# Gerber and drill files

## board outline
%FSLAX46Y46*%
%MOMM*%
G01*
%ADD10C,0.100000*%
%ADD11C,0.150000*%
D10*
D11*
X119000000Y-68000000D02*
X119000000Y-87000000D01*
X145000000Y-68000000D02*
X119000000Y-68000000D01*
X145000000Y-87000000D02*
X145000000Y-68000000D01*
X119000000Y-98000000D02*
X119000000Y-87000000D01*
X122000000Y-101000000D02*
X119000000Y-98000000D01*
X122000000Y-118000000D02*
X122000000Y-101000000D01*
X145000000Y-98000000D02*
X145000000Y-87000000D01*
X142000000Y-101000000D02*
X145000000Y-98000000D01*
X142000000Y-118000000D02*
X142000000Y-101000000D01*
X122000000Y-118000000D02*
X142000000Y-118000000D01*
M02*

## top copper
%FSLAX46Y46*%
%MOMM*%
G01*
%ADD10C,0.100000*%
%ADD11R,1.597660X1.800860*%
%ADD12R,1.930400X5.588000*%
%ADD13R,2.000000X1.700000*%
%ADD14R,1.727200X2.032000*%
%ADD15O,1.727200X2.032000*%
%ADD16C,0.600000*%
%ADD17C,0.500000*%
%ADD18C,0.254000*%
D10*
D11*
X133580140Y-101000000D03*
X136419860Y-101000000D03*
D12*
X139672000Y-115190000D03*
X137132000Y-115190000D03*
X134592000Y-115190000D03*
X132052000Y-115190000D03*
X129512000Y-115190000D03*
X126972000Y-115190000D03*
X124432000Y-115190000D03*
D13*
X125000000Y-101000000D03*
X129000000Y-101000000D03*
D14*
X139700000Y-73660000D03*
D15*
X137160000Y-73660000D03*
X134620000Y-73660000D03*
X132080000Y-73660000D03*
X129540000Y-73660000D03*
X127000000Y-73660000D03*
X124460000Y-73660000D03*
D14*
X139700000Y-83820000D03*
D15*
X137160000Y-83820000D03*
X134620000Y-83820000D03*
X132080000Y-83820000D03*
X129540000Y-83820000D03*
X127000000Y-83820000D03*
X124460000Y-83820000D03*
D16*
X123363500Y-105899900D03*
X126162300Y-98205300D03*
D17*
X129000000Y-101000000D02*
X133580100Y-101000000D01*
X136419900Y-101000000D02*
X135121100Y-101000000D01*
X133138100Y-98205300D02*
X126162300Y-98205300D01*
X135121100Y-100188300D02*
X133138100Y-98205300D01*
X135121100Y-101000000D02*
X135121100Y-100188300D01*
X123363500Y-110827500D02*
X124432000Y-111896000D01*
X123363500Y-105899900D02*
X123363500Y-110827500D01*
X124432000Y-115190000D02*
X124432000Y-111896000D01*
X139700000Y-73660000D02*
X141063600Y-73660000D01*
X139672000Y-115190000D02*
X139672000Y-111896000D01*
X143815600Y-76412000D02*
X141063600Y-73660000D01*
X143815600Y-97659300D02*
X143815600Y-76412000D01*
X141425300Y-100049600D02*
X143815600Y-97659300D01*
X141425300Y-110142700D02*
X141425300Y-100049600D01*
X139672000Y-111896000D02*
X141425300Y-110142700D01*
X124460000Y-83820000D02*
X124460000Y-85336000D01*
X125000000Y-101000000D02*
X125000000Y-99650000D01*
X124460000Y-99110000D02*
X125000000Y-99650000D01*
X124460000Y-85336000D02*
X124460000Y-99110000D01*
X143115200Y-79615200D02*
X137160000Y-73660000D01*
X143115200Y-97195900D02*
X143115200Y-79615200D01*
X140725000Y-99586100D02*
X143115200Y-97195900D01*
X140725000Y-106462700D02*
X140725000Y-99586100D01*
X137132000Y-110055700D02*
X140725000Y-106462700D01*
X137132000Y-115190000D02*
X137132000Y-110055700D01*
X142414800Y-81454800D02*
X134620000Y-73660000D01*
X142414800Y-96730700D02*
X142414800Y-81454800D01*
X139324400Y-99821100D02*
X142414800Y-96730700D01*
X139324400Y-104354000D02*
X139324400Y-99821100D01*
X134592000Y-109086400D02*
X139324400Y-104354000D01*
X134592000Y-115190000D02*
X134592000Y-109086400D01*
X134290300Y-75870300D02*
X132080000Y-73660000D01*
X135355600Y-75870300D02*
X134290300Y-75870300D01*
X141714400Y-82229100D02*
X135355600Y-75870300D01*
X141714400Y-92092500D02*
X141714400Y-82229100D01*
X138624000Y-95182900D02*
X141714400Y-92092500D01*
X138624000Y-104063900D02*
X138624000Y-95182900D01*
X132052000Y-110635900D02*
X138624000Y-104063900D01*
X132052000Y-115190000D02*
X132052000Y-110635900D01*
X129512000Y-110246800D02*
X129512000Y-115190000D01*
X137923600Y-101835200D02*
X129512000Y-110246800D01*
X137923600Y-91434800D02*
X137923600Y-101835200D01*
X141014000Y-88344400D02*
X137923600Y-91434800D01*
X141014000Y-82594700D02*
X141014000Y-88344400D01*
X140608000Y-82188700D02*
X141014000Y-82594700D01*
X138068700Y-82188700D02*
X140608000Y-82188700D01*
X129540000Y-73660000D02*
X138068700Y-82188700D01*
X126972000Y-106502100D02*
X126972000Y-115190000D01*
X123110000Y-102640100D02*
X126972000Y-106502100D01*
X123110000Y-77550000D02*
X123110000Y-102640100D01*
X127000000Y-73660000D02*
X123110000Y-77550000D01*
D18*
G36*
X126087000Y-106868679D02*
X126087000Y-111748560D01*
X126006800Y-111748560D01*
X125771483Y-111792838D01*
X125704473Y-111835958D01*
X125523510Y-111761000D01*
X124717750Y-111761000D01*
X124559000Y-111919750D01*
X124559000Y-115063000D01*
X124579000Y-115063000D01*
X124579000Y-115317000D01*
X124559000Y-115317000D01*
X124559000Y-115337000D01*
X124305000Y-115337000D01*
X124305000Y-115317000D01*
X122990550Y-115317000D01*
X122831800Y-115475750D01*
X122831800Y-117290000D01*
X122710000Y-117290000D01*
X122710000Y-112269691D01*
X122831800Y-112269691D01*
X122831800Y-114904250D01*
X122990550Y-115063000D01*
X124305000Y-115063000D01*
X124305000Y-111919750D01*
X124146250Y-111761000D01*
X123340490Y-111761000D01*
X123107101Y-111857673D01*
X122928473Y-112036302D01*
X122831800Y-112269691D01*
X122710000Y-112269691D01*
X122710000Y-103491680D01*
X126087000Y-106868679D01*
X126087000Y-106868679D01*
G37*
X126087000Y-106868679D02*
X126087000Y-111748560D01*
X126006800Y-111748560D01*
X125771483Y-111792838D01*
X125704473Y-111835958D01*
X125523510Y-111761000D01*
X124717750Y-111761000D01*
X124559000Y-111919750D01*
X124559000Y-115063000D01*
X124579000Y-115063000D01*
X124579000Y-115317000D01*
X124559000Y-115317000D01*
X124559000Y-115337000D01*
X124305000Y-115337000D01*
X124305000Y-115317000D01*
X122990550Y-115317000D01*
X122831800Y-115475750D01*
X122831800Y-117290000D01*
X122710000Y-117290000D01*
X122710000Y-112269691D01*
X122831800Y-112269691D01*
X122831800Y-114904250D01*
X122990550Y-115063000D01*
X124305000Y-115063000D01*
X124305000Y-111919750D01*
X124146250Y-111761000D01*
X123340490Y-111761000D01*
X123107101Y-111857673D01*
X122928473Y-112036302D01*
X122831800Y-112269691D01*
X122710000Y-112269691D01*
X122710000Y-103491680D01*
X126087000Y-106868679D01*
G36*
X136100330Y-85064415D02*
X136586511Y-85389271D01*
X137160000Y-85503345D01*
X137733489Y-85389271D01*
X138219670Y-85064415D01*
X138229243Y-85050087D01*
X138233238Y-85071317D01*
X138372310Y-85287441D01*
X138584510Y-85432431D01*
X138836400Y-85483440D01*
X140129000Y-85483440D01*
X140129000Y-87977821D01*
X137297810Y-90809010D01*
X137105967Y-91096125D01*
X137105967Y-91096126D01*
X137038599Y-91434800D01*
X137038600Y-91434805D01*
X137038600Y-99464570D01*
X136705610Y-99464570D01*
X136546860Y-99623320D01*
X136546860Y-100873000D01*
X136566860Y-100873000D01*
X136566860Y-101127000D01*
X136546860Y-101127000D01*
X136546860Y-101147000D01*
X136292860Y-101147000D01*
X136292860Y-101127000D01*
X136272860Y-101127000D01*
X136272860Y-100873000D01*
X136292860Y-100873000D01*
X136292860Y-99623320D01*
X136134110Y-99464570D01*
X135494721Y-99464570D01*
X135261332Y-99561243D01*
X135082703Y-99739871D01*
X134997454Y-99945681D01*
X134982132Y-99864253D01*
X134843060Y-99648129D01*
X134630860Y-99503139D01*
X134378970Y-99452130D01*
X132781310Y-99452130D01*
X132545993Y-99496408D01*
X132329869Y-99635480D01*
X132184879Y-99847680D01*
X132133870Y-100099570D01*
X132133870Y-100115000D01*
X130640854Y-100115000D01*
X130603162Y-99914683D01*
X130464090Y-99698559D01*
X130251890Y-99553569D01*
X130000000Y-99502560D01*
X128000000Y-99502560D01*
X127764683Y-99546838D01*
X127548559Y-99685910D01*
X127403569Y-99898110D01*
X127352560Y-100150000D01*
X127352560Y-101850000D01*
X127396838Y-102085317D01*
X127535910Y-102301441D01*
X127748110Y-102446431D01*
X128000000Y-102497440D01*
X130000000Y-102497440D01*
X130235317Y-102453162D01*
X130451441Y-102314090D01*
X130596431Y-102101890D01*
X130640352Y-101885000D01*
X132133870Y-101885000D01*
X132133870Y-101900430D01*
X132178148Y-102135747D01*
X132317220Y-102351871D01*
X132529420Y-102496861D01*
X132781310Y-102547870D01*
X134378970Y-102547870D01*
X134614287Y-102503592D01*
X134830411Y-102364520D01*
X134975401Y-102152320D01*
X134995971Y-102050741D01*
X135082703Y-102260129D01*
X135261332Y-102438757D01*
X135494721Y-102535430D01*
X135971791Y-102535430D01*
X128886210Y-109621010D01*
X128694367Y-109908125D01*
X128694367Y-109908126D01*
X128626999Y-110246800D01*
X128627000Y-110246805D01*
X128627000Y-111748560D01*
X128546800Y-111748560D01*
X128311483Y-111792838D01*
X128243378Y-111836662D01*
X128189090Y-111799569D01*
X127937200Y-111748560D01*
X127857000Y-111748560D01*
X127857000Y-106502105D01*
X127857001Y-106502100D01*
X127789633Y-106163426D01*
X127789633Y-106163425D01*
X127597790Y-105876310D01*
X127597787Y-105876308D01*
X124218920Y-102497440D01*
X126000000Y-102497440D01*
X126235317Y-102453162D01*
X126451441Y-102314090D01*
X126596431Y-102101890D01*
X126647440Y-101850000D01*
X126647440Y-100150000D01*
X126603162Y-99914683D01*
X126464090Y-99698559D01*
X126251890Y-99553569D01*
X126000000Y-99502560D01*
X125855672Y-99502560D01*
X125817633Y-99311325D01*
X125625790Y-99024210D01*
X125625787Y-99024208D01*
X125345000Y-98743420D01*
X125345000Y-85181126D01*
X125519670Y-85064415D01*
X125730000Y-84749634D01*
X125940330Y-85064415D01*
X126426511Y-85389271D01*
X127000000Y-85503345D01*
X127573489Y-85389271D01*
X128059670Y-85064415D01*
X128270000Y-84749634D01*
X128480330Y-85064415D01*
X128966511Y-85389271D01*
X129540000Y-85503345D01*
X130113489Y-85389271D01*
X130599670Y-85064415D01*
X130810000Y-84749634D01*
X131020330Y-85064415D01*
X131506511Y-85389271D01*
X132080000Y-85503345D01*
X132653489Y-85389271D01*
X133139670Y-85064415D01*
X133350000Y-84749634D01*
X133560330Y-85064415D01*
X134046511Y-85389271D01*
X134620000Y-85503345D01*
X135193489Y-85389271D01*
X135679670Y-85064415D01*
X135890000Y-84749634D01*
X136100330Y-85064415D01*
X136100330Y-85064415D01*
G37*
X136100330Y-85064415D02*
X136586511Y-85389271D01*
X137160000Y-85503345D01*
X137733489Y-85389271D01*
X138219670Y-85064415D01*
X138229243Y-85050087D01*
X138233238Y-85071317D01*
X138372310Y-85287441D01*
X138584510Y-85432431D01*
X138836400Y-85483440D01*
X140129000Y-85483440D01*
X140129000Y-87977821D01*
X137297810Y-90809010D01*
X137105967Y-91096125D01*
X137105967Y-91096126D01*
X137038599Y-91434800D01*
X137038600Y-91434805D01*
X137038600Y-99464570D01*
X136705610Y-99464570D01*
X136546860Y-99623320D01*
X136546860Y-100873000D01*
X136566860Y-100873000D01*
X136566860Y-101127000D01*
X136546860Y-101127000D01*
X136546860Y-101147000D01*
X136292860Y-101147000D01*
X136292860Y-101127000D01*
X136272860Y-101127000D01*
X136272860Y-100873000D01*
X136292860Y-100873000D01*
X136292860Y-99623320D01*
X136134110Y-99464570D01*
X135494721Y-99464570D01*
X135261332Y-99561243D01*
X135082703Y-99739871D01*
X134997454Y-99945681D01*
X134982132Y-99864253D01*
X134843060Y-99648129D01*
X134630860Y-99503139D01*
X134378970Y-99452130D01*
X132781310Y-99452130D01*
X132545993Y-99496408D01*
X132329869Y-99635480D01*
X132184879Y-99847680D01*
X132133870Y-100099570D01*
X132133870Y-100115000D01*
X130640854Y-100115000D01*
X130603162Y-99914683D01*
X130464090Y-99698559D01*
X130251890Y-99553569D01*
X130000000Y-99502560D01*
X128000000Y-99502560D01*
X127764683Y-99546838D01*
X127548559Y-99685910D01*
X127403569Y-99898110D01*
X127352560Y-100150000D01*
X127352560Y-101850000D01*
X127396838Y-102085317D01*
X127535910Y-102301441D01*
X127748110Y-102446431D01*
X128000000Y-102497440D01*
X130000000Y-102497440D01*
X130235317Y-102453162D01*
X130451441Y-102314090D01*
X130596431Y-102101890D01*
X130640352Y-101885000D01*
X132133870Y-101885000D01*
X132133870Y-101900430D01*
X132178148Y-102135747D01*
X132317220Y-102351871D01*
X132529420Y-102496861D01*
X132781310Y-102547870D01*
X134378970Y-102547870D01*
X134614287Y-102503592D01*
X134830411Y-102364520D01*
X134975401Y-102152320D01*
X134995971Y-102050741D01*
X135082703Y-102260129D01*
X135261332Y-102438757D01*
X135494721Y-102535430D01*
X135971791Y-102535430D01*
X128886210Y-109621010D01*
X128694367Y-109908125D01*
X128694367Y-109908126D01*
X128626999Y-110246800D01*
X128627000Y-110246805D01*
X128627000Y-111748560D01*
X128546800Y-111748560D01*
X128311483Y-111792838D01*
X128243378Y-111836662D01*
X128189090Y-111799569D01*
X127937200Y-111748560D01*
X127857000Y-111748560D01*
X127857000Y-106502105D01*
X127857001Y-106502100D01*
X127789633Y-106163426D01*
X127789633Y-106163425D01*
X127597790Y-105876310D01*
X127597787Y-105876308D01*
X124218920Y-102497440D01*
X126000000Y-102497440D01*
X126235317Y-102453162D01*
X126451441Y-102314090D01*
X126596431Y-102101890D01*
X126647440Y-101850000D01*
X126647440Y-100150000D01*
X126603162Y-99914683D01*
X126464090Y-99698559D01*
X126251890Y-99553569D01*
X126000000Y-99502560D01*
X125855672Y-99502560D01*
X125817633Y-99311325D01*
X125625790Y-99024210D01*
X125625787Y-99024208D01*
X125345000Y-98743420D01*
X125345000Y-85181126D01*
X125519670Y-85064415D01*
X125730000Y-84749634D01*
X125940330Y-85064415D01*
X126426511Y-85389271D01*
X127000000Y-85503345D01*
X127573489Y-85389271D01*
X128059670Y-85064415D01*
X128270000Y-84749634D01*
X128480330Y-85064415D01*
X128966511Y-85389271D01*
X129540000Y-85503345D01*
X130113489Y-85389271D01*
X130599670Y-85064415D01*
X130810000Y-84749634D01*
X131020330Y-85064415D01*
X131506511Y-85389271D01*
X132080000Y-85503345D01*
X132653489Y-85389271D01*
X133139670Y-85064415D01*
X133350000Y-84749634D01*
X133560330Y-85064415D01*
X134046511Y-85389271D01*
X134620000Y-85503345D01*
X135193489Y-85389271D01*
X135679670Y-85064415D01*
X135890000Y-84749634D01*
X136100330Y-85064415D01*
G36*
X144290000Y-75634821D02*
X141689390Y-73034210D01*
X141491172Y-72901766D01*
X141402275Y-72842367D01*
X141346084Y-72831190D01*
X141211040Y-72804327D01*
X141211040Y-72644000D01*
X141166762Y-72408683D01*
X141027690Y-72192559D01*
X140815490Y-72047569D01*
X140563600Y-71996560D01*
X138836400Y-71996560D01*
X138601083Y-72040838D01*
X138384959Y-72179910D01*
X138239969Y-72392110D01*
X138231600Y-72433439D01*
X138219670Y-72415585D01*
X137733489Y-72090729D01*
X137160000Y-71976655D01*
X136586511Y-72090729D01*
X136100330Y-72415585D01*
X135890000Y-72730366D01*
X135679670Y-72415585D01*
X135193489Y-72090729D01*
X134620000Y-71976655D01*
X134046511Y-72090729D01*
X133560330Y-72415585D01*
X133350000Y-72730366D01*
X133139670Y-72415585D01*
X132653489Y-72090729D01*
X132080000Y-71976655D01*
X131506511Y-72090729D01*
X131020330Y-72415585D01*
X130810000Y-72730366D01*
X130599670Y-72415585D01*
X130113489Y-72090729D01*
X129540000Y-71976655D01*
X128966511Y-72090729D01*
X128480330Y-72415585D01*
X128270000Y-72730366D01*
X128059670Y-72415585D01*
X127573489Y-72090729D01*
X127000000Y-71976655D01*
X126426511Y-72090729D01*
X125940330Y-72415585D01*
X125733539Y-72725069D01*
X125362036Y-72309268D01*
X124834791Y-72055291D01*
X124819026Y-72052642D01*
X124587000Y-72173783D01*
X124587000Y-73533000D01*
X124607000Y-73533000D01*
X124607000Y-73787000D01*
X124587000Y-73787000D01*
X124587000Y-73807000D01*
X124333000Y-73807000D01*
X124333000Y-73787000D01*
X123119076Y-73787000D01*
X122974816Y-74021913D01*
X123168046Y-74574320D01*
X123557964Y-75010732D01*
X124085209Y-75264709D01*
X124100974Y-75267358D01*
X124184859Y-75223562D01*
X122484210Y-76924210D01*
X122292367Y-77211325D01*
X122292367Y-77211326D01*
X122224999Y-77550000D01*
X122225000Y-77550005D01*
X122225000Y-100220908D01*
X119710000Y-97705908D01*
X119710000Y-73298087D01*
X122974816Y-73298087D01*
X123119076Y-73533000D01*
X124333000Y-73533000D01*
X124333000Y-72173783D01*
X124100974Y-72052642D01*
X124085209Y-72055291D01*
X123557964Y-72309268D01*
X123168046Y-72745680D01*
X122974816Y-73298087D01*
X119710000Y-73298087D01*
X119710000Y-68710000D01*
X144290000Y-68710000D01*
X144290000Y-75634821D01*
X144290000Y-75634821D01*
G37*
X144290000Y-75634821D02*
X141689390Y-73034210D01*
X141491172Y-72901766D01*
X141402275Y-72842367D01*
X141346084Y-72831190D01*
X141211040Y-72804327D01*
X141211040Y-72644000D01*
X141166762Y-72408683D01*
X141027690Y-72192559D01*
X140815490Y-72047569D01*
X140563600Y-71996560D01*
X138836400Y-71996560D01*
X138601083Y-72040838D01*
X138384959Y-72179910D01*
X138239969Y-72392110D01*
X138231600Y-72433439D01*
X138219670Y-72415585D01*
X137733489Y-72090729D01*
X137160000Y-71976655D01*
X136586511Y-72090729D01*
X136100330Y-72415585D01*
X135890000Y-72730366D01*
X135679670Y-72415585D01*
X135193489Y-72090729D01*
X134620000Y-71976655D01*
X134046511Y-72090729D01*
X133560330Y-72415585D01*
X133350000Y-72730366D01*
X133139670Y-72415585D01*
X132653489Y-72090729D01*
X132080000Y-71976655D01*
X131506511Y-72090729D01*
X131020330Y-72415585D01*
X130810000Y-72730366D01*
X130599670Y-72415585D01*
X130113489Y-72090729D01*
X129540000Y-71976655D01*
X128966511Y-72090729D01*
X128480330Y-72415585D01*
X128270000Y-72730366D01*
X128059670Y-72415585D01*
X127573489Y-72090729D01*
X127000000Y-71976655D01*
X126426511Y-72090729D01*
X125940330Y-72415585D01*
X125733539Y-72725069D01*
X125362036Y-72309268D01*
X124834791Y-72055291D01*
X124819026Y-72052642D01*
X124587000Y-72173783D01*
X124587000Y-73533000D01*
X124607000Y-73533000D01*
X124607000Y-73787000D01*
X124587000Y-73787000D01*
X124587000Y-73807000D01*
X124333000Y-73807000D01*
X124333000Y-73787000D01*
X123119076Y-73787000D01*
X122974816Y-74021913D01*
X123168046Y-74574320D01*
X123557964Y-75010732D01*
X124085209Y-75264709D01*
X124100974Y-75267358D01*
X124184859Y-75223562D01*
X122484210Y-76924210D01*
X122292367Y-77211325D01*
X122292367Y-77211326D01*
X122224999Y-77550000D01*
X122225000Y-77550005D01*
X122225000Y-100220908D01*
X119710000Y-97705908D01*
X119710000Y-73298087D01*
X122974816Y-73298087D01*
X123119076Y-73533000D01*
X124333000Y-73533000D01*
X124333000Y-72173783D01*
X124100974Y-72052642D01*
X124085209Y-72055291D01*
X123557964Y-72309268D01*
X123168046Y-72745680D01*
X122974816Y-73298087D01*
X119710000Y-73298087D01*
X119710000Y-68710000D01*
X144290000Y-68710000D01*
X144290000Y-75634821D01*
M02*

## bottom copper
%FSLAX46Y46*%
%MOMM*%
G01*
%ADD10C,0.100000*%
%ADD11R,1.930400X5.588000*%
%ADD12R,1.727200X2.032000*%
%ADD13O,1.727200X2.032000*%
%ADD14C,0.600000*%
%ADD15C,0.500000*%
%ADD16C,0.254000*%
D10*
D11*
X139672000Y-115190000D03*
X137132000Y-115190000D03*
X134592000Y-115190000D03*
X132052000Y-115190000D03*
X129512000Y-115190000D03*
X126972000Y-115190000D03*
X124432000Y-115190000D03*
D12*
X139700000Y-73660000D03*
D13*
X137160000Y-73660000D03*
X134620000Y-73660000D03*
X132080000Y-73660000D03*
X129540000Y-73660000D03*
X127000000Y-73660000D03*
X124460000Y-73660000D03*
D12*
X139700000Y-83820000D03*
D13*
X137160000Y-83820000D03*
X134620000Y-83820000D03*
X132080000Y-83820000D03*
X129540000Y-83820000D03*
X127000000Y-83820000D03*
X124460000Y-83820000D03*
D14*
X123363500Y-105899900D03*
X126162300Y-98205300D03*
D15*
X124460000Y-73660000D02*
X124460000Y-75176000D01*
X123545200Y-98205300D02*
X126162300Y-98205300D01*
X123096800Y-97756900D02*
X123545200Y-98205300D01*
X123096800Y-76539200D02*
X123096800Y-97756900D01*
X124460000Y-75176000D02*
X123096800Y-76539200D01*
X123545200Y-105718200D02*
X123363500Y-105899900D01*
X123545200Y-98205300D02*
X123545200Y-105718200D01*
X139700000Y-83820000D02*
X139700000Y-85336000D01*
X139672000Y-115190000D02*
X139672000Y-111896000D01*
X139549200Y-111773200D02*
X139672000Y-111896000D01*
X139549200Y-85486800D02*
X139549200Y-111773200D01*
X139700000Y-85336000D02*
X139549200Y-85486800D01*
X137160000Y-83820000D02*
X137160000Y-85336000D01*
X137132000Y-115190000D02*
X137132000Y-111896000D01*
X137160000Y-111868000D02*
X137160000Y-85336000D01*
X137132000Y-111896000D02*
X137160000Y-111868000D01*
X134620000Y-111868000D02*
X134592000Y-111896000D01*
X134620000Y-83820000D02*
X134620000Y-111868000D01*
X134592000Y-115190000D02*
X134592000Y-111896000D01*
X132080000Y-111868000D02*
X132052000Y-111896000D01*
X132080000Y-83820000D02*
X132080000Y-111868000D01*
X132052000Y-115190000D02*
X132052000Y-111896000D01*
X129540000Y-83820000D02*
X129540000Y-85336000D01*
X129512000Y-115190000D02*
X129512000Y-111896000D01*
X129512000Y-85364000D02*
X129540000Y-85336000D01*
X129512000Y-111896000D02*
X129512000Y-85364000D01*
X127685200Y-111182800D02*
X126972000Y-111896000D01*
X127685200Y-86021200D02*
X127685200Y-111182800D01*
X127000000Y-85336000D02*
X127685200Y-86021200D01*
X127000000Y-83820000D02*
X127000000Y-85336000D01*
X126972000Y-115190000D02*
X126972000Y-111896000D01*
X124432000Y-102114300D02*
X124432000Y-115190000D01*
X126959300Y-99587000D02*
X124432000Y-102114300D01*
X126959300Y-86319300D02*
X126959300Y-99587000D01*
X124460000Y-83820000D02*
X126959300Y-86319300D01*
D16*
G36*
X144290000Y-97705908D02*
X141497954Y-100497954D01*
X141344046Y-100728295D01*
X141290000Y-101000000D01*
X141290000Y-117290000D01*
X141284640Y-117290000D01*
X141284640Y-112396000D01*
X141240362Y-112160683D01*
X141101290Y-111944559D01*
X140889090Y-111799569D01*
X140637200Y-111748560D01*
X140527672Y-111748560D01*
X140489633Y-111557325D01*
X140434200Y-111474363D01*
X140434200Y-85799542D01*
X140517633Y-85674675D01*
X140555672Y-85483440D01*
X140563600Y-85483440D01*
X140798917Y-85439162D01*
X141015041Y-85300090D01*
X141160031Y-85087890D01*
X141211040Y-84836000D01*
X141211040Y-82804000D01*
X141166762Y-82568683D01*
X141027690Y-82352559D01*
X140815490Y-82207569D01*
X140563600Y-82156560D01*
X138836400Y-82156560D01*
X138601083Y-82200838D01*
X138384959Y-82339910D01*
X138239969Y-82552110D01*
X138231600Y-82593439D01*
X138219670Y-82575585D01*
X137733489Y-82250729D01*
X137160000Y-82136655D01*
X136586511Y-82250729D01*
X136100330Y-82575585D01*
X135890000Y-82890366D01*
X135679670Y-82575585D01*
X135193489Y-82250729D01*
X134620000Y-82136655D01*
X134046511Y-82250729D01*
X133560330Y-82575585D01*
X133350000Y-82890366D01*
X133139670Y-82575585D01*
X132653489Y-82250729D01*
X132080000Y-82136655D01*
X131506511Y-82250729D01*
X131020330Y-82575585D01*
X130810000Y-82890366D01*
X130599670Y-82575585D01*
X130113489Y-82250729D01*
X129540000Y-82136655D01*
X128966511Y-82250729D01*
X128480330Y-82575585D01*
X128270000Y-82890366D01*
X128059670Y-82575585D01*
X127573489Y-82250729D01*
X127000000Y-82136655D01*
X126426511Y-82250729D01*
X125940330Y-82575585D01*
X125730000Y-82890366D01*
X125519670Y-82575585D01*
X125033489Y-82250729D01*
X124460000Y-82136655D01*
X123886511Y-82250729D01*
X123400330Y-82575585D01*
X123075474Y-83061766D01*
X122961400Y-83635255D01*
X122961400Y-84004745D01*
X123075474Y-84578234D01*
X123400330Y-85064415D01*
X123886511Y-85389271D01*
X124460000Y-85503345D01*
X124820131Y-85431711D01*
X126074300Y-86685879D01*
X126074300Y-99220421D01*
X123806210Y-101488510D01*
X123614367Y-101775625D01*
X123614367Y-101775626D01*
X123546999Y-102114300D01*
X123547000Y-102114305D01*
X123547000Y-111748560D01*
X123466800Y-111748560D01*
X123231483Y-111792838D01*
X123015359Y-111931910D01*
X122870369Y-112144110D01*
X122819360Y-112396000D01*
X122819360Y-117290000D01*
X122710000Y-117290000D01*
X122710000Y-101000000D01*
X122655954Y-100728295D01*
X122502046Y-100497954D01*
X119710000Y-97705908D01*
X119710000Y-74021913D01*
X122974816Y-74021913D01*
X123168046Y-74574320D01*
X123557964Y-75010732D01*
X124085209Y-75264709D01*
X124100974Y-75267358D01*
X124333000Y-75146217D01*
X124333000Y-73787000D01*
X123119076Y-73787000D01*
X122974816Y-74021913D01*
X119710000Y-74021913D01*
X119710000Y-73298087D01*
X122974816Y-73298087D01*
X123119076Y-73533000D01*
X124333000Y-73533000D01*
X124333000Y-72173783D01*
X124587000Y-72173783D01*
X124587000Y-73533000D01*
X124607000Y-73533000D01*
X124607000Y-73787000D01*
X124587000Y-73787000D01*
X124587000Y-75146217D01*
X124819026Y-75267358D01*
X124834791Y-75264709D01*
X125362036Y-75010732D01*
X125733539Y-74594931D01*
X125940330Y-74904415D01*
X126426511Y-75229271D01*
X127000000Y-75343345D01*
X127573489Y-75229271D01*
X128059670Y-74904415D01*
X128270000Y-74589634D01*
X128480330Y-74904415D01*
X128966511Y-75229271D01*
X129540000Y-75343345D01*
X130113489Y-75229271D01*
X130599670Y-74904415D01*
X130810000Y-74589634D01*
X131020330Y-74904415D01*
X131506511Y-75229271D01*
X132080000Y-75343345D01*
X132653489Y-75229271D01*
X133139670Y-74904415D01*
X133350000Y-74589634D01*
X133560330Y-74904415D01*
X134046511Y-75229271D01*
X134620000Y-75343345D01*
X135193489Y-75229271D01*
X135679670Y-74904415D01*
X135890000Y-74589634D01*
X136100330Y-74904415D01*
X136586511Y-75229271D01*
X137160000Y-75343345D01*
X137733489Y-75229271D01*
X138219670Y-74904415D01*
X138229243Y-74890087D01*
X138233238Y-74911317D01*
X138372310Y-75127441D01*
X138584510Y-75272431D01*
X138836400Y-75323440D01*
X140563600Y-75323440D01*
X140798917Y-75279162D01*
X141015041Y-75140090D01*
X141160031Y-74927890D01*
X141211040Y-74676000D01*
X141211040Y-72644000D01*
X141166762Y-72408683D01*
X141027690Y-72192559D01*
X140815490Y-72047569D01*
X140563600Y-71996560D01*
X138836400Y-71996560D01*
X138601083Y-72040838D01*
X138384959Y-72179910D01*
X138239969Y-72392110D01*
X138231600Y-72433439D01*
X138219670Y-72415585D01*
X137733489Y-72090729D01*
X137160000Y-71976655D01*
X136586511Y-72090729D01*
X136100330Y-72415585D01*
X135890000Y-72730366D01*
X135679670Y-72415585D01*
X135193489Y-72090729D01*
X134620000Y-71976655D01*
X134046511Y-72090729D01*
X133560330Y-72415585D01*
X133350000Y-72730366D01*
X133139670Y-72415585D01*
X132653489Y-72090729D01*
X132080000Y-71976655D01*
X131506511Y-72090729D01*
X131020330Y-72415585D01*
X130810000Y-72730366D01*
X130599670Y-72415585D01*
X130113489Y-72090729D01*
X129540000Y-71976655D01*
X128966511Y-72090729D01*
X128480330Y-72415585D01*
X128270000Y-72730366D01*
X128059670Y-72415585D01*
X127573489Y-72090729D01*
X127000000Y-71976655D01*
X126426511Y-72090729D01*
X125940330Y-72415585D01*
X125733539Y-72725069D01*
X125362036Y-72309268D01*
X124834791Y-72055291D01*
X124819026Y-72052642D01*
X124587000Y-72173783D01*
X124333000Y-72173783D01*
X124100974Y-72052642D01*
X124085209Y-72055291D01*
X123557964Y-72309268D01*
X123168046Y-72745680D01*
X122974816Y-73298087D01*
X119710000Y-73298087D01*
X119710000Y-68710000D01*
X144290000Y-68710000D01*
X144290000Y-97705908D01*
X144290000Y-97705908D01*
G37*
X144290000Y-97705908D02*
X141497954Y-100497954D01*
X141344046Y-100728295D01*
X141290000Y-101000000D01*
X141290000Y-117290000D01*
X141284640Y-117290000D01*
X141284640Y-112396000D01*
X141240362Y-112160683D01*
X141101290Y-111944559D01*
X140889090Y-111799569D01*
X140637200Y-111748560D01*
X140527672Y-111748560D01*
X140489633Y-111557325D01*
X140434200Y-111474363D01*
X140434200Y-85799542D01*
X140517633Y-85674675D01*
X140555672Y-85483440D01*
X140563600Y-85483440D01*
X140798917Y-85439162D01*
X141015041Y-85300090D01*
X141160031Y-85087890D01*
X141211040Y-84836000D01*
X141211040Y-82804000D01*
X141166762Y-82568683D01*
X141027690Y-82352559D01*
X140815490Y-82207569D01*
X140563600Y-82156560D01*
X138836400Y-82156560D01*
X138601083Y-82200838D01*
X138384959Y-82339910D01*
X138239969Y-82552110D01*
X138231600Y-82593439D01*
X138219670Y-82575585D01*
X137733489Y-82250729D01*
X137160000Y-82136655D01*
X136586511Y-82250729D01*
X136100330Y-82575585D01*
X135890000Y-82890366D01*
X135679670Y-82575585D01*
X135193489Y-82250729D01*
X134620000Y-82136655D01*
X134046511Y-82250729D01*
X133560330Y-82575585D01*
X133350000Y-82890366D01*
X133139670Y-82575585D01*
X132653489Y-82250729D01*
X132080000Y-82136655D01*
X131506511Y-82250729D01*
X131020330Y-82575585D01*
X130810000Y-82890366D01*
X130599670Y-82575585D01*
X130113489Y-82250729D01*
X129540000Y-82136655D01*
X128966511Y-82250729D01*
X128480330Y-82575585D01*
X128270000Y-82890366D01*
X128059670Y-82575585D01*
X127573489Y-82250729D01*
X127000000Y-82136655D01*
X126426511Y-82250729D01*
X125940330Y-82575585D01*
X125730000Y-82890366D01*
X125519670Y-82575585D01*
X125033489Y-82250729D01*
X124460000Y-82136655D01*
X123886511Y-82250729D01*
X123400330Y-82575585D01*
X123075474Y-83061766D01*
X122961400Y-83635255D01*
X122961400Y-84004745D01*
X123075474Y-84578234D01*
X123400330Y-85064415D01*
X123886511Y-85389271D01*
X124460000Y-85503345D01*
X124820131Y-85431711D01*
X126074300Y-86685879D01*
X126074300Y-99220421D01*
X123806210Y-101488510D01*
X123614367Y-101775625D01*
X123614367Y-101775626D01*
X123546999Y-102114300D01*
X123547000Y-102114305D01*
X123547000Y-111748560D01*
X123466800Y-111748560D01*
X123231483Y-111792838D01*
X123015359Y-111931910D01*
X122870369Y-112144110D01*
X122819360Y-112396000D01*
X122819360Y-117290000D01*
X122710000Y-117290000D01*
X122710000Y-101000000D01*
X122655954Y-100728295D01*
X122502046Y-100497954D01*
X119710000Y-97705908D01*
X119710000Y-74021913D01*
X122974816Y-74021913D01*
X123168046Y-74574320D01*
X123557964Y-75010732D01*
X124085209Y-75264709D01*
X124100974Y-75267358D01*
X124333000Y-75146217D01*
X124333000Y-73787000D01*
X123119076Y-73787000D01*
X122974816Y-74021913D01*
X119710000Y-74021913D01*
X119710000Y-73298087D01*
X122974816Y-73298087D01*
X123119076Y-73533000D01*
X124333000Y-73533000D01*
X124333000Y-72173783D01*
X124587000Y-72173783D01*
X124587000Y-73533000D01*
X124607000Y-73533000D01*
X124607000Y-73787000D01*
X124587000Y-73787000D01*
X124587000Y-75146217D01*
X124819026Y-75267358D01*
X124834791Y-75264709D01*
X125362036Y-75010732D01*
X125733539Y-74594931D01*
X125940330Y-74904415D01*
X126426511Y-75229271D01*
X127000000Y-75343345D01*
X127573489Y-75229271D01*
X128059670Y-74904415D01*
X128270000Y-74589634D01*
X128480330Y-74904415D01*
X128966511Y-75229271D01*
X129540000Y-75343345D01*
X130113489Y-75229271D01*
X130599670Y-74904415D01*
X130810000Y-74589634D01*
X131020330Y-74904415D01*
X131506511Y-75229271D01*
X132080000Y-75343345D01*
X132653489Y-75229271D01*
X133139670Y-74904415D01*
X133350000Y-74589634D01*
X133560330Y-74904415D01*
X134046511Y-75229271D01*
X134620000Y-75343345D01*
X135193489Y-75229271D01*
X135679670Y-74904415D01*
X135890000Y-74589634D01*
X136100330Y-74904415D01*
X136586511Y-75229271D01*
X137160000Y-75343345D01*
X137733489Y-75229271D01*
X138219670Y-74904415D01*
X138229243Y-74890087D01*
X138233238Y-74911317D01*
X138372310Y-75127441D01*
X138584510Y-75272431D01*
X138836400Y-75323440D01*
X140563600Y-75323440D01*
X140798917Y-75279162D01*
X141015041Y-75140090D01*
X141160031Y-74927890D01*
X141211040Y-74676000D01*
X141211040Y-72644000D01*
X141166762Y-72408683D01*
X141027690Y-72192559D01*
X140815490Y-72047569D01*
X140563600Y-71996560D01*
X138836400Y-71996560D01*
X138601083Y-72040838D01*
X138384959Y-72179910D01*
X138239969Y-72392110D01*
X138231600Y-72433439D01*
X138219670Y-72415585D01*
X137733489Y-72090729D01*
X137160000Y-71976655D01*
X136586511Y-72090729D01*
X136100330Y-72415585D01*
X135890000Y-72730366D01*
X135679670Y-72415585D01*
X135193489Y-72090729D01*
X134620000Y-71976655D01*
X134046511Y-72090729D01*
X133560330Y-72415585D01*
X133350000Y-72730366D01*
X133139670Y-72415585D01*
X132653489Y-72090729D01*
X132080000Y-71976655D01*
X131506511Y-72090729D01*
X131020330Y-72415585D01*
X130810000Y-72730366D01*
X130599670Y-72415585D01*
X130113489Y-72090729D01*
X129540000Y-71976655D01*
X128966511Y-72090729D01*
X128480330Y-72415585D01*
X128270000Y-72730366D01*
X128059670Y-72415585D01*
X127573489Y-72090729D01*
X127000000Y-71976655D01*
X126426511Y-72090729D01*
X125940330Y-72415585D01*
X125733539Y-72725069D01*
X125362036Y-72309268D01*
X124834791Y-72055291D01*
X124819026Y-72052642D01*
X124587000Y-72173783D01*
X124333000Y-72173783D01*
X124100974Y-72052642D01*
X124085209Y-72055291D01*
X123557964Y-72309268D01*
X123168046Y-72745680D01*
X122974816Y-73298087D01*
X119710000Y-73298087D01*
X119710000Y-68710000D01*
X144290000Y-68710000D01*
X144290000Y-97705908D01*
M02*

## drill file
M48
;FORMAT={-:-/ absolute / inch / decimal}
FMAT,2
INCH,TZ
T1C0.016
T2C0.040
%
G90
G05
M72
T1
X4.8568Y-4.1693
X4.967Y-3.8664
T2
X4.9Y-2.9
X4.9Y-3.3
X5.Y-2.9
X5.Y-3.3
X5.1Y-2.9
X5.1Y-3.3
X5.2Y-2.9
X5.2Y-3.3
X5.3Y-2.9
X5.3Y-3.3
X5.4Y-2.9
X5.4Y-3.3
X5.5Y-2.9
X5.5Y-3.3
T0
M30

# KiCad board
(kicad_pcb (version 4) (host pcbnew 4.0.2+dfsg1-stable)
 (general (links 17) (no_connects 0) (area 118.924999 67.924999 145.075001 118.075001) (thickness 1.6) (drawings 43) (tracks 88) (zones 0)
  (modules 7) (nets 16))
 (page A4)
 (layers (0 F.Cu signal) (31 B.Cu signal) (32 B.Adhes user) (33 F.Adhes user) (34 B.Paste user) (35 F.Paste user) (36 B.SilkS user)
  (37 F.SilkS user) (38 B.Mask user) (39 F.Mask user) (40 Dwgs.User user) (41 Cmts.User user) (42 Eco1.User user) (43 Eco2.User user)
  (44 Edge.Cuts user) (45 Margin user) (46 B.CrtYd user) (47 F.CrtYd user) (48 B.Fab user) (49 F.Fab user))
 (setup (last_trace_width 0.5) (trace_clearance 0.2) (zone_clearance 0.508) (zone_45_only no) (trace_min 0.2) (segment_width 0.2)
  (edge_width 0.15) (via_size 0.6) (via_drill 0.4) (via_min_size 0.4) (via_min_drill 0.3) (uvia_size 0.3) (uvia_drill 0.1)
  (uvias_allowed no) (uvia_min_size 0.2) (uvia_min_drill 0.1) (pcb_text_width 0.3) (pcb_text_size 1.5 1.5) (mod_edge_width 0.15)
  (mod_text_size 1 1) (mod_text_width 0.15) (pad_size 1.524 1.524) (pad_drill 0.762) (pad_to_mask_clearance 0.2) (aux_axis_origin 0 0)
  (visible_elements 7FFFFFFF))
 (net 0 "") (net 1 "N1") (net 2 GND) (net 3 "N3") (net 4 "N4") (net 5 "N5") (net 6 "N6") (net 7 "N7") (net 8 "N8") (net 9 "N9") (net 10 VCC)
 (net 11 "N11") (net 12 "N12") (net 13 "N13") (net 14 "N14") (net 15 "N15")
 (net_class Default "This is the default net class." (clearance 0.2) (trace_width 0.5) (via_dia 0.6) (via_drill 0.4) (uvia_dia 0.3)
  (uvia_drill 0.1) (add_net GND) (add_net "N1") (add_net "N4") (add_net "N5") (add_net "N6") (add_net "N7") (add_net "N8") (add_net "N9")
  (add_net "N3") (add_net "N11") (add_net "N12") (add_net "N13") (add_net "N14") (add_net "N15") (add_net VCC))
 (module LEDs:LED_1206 (layer F.Cu) (at 135 101 180)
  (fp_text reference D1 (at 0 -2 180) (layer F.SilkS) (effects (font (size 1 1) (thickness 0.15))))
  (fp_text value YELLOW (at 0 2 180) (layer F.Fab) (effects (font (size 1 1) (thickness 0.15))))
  (pad 2 smd rect (at 1.41986 0) (size 1.59766 1.80086) (layers F.Cu F.Paste F.Mask) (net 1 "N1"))
  (pad 1 smd rect (at -1.41986 0) (size 1.59766 1.80086) (layers F.Cu F.Paste F.Mask) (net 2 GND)))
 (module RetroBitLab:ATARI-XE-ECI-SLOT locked (layer F.Cu) (at 122.4 119)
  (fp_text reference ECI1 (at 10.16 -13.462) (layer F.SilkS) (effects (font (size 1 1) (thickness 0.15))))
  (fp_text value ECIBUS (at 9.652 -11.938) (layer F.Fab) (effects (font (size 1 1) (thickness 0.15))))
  (pad A smd rect (at 17.272 -3.81 270) (size 5.588 1.9304) (layers F.Cu F.Paste F.Mask) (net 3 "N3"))
  (pad 1 smd rect (at 17.272 -3.81 270) (size 5.588 1.9304) (layers B.Cu B.Paste B.Mask) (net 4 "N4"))
  (pad 2 smd rect (at 14.732 -3.81 270) (size 5.588 1.9304) (layers B.Cu B.Paste B.Mask) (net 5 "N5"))
  (pad 3 smd rect (at 12.192 -3.81 270) (size 5.588 1.9304) (layers B.Cu B.Paste B.Mask) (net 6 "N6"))
  (pad 4 smd rect (at 9.652 -3.81 270) (size 5.588 1.9304) (layers B.Cu B.Paste B.Mask) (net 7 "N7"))
  (pad 5 smd rect (at 7.112 -3.81 270) (size 5.588 1.9304) (layers B.Cu B.Paste B.Mask) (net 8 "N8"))
  (pad 6 smd rect (at 4.572 -3.81 270) (size 5.588 1.9304) (layers B.Cu B.Paste B.Mask) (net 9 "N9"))
  (pad 7 smd rect (at 2.032 -3.81 270) (size 5.588 1.9304) (layers B.Cu B.Paste B.Mask) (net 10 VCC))
  (pad B smd rect (at 14.732 -3.81 270) (size 5.588 1.9304) (layers F.Cu F.Paste F.Mask) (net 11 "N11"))
  (pad C smd rect (at 12.192 -3.81 270) (size 5.588 1.9304) (layers F.Cu F.Paste F.Mask) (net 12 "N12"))
  (pad D smd rect (at 9.652 -3.81 270) (size 5.588 1.9304) (layers F.Cu F.Paste F.Mask) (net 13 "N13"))
  (pad E smd rect (at 7.112 -3.81 270) (size 5.588 1.9304) (layers F.Cu F.Paste F.Mask) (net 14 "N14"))
  (pad F smd rect (at 4.572 -3.81 270) (size 5.588 1.9304) (layers F.Cu F.Paste F.Mask) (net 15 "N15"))
  (pad H smd rect (at 2.032 -3.81 270) (size 5.588 1.9304) (layers F.Cu F.Paste F.Mask) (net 2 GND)))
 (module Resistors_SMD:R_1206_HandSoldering (layer F.Cu) (at 127 101)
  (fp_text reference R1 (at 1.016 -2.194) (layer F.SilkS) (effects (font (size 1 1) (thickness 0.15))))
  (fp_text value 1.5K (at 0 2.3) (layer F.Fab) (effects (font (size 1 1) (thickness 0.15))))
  (pad 1 smd rect (at -2 0) (size 2 1.7) (layers F.Cu F.Paste F.Mask) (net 10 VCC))
  (pad 2 smd rect (at 2 0) (size 2 1.7) (layers F.Cu F.Paste F.Mask) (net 1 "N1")))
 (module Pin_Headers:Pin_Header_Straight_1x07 (layer F.Cu) (at 139.7 73.66 270)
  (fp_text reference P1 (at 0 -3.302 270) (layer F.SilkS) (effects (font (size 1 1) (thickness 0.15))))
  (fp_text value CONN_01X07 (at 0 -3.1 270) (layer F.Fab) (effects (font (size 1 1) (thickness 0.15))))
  (pad 1 thru_hole rect (at 0 0 270) (size 2.032 1.7272) (drill 1.016) (layers *.Cu *.Mask F.SilkS) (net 3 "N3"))
  (pad 2 thru_hole oval (at 0 2.54 270) (size 2.032 1.7272) (drill 1.016) (layers *.Cu *.Mask F.SilkS) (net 11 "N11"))
  (pad 3 thru_hole oval (at 0 5.08 270) (size 2.032 1.7272) (drill 1.016) (layers *.Cu *.Mask F.SilkS) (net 12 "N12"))
  (pad 4 thru_hole oval (at 0 7.62 270) (size 2.032 1.7272) (drill 1.016) (layers *.Cu *.Mask F.SilkS) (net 13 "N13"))
  (pad 5 thru_hole oval (at 0 10.16 270) (size 2.032 1.7272) (drill 1.016) (layers *.Cu *.Mask F.SilkS) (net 14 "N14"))
  (pad 6 thru_hole oval (at 0 12.7 270) (size 2.032 1.7272) (drill 1.016) (layers *.Cu *.Mask F.SilkS) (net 15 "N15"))
  (pad 7 thru_hole oval (at 0 15.24 270) (size 2.032 1.7272) (drill 1.016) (layers *.Cu *.Mask F.SilkS) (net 2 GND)))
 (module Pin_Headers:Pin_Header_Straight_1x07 (layer F.Cu) (at 139.7 83.82 270)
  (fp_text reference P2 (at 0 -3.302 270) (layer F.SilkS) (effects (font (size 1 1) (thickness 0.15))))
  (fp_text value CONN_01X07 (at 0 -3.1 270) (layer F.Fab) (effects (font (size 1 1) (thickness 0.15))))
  (pad 1 thru_hole rect (at 0 0 270) (size 2.032 1.7272) (drill 1.016) (layers *.Cu *.Mask F.SilkS) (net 4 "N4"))
  (pad 2 thru_hole oval (at 0 2.54 270) (size 2.032 1.7272) (drill 1.016) (layers *.Cu *.Mask F.SilkS) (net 5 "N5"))
  (pad 3 thru_hole oval (at 0 5.08 270) (size 2.032 1.7272) (drill 1.016) (layers *.Cu *.Mask F.SilkS) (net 6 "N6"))
  (pad 4 thru_hole oval (at 0 7.62 270) (size 2.032 1.7272) (drill 1.016) (layers *.Cu *.Mask F.SilkS) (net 7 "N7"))
  (pad 5 thru_hole oval (at 0 10.16 270) (size 2.032 1.7272) (drill 1.016) (layers *.Cu *.Mask F.SilkS) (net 8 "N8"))
  (pad 6 thru_hole oval (at 0 12.7 270) (size 2.032 1.7272) (drill 1.016) (layers *.Cu *.Mask F.SilkS) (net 9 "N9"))
  (pad 7 thru_hole oval (at 0 15.24 270) (size 2.032 1.7272) (drill 1.016) (layers *.Cu *.Mask F.SilkS) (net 10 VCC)))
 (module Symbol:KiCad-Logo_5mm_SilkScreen (layer B.Cu) (at 132.08 91.948 180)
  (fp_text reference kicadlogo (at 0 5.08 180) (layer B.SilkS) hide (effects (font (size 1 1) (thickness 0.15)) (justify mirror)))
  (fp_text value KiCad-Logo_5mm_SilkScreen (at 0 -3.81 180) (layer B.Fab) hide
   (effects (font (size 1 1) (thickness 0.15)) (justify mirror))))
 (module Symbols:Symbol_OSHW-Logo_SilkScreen (layer B.Cu) (at 132.588 97.028 180)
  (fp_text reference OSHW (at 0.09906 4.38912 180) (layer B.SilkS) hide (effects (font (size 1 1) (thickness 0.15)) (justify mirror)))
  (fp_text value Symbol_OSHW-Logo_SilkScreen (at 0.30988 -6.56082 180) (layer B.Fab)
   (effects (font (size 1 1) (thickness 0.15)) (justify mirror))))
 (gr_line (start 119 68) (end 119 87) (angle 90) (layer Edge.Cuts) (width 0.15))
 (gr_line (start 145 68) (end 119 68) (angle 90) (layer Edge.Cuts) (width 0.15))
 (gr_line (start 145 87) (end 145 68) (angle 90) (layer Edge.Cuts) (width 0.15))
 (gr_line (start 119 98) (end 119 87) (angle 90) (layer Edge.Cuts) (width 0.15))
 (gr_line (start 122 101) (end 119 98) (angle 90) (layer Edge.Cuts) (width 0.15))
 (gr_line (start 122 118) (end 122 101) (angle 90) (layer Edge.Cuts) (width 0.15))
 (gr_line (start 145 98) (end 145 87) (angle 90) (layer Edge.Cuts) (width 0.15))
 (gr_line (start 142 101) (end 145 98) (angle 90) (layer Edge.Cuts) (width 0.15))
 (gr_line (start 142 118) (end 142 101) (angle 90) (layer Edge.Cuts) (width 0.15))
 (gr_line (start 122 118) (end 142 118) (angle 90) (layer Edge.Cuts) (width 0.15))
 (segment (start 129 101) (end 133.5801 101) (width 0.5) (layer F.Cu) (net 1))
 (via (at 123.3635 105.8999) (size 0.6) (layers F.Cu B.Cu) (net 2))
 (via (at 126.1623 98.2053) (size 0.6) (layers F.Cu B.Cu) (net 2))
 (segment (start 124.46 73.66) (end 124.46 75.176) (width 0.5) (layer B.Cu) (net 2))
 (segment (start 136.4199 101) (end 135.1211 101) (width 0.5) (layer F.Cu) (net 2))
 (segment (start 133.1381 98.2053) (end 126.1623 98.2053) (width 0.5) (layer F.Cu) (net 2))
 (segment (start 135.1211 100.1883) (end 133.1381 98.2053) (width 0.5) (layer F.Cu) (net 2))
 (segment (start 135.1211 101) (end 135.1211 100.1883) (width 0.5) (layer F.Cu) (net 2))
 (segment (start 123.5452 98.2053) (end 126.1623 98.2053) (width 0.5) (layer B.Cu) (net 2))
 (segment (start 123.0968 97.7569) (end 123.5452 98.2053) (width 0.5) (layer B.Cu) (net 2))
 (segment (start 123.0968 76.5392) (end 123.0968 97.7569) (width 0.5) (layer B.Cu) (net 2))
 (segment (start 124.46 75.176) (end 123.0968 76.5392) (width 0.5) (layer B.Cu) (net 2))
 (segment (start 123.5452 105.7182) (end 123.3635 105.8999) (width 0.5) (layer B.Cu) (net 2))
 (segment (start 123.5452 98.2053) (end 123.5452 105.7182) (width 0.5) (layer B.Cu) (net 2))
 (segment (start 123.3635 110.8275) (end 124.432 111.896) (width 0.5) (layer F.Cu) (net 2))
 (segment (start 123.3635 105.8999) (end 123.3635 110.8275) (width 0.5) (layer F.Cu) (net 2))
 (segment (start 124.432 115.19) (end 124.432 111.896) (width 0.5) (layer F.Cu) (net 2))
 (segment (start 139.7 73.66) (end 141.0636 73.66) (width 0.5) (layer F.Cu) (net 3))
 (segment (start 139.672 115.19) (end 139.672 111.896) (width 0.5) (layer F.Cu) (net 3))
 (segment (start 143.8156 76.412) (end 141.0636 73.66) (width 0.5) (layer F.Cu) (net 3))
 (segment (start 143.8156 97.6593) (end 143.8156 76.412) (width 0.5) (layer F.Cu) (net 3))
 (segment (start 141.4253 100.0496) (end 143.8156 97.6593) (width 0.5) (layer F.Cu) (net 3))
 (segment (start 141.4253 110.1427) (end 141.4253 100.0496) (width 0.5) (layer F.Cu) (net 3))
 (segment (start 139.672 111.896) (end 141.4253 110.1427) (width 0.5) (layer F.Cu) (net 3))
 (segment (start 139.7 83.82) (end 139.7 85.336) (width 0.5) (layer B.Cu) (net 4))
 (segment (start 139.672 115.19) (end 139.672 111.896) (width 0.5) (layer B.Cu) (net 4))
 (segment (start 139.5492 111.7732) (end 139.672 111.896) (width 0.5) (layer B.Cu) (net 4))
 (segment (start 139.5492 85.4868) (end 139.5492 111.7732) (width 0.5) (layer B.Cu) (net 4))
 (segment (start 139.7 85.336) (end 139.5492 85.4868) (width 0.5) (layer B.Cu) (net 4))
 (segment (start 137.16 83.82) (end 137.16 85.336) (width 0.5) (layer B.Cu) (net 5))
 (segment (start 137.132 115.19) (end 137.132 111.896) (width 0.5) (layer B.Cu) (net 5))
 (segment (start 137.16 111.868) (end 137.16 85.336) (width 0.5) (layer B.Cu) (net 5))
 (segment (start 137.132 111.896) (end 137.16 111.868) (width 0.5) (layer B.Cu) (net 5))
 (segment (start 134.62 111.868) (end 134.592 111.896) (width 0.5) (layer B.Cu) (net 6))
 (segment (start 134.62 83.82) (end 134.62 111.868) (width 0.5) (layer B.Cu) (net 6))
 (segment (start 134.592 115.19) (end 134.592 111.896) (width 0.5) (layer B.Cu) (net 6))
 (segment (start 132.08 111.868) (end 132.052 111.896) (width 0.5) (layer B.Cu) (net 7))
 (segment (start 132.08 83.82) (end 132.08 111.868) (width 0.5) (layer B.Cu) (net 7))
 (segment (start 132.052 115.19) (end 132.052 111.896) (width 0.5) (layer B.Cu) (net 7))
 (segment (start 129.54 83.82) (end 129.54 85.336) (width 0.5) (layer B.Cu) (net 8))
 (segment (start 129.512 115.19) (end 129.512 111.896) (width 0.5) (layer B.Cu) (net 8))
 (segment (start 129.512 85.364) (end 129.54 85.336) (width 0.5) (layer B.Cu) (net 8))
 (segment (start 129.512 111.896) (end 129.512 85.364) (width 0.5) (layer B.Cu) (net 8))
 (segment (start 127.6852 111.1828) (end 126.972 111.896) (width 0.5) (layer B.Cu) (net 9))
 (segment (start 127.6852 86.0212) (end 127.6852 111.1828) (width 0.5) (layer B.Cu) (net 9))
 (segment (start 127 85.336) (end 127.6852 86.0212) (width 0.5) (layer B.Cu) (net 9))
 (segment (start 127 83.82) (end 127 85.336) (width 0.5) (layer B.Cu) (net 9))
 (segment (start 126.972 115.19) (end 126.972 111.896) (width 0.5) (layer B.Cu) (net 9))
 (segment (start 124.46 83.82) (end 124.46 85.336) (width 0.5) (layer F.Cu) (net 10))
 (segment (start 125 101) (end 125 99.65) (width 0.5) (layer F.Cu) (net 10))
 (segment (start 124.46 99.11) (end 125 99.65) (width 0.5) (layer F.Cu) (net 10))
 (segment (start 124.46 85.336) (end 124.46 99.11) (width 0.5) (layer F.Cu) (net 10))
 (segment (start 124.432 102.1143) (end 124.432 115.19) (width 0.5) (layer B.Cu) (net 10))
 (segment (start 126.9593 99.587) (end 124.432 102.1143) (width 0.5) (layer B.Cu) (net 10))
 (segment (start 126.9593 86.3193) (end 126.9593 99.587) (width 0.5) (layer B.Cu) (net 10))
 (segment (start 124.46 83.82) (end 126.9593 86.3193) (width 0.5) (layer B.Cu) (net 10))
 (segment (start 143.1152 79.6152) (end 137.16 73.66) (width 0.5) (layer F.Cu) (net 11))
 (segment (start 143.1152 97.1959) (end 143.1152 79.6152) (width 0.5) (layer F.Cu) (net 11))
 (segment (start 140.725 99.5861) (end 143.1152 97.1959) (width 0.5) (layer F.Cu) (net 11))
 (segment (start 140.725 106.4627) (end 140.725 99.5861) (width 0.5) (layer F.Cu) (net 11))
 (segment (start 137.132 110.0557) (end 140.725 106.4627) (width 0.5) (layer F.Cu) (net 11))
 (segment (start 137.132 115.19) (end 137.132 110.0557) (width 0.5) (layer F.Cu) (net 11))
 (segment (start 142.4148 81.4548) (end 134.62 73.66) (width 0.5) (layer F.Cu) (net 12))
 (segment (start 142.4148 96.7307) (end 142.4148 81.4548) (width 0.5) (layer F.Cu) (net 12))
 (segment (start 139.3244 99.8211) (end 142.4148 96.7307) (width 0.5) (layer F.Cu) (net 12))
 (segment (start 139.3244 104.354) (end 139.3244 99.8211) (width 0.5) (layer F.Cu) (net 12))
 (segment (start 134.592 109.0864) (end 139.3244 104.354) (width 0.5) (layer F.Cu) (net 12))
 (segment (start 134.592 115.19) (end 134.592 109.0864) (width 0.5) (layer F.Cu) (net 12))
 (segment (start 134.2903 75.8703) (end 132.08 73.66) (width 0.5) (layer F.Cu) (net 13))
 (segment (start 135.3556 75.8703) (end 134.2903 75.8703) (width 0.5) (layer F.Cu) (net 13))
 (segment (start 141.7144 82.2291) (end 135.3556 75.8703) (width 0.5) (layer F.Cu) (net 13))
 (segment (start 141.7144 92.0925) (end 141.7144 82.2291) (width 0.5) (layer F.Cu) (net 13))
 (segment (start 138.624 95.1829) (end 141.7144 92.0925) (width 0.5) (layer F.Cu) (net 13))
 (segment (start 138.624 104.0639) (end 138.624 95.1829) (width 0.5) (layer F.Cu) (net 13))
 (segment (start 132.052 110.6359) (end 138.624 104.0639) (width 0.5) (layer F.Cu) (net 13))
 (segment (start 132.052 115.19) (end 132.052 110.6359) (width 0.5) (layer F.Cu) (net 13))
 (segment (start 129.512 110.2468) (end 129.512 115.19) (width 0.5) (layer F.Cu) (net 14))
 (segment (start 137.9236 101.8352) (end 129.512 110.2468) (width 0.5) (layer F.Cu) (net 14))
 (segment (start 137.9236 91.4348) (end 137.9236 101.8352) (width 0.5) (layer F.Cu) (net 14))
 (segment (start 141.014 88.3444) (end 137.9236 91.4348) (width 0.5) (layer F.Cu) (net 14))
 (segment (start 141.014 82.5947) (end 141.014 88.3444) (width 0.5) (layer F.Cu) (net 14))
 (segment (start 140.608 82.1887) (end 141.014 82.5947) (width 0.5) (layer F.Cu) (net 14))
 (segment (start 138.0687 82.1887) (end 140.608 82.1887) (width 0.5) (layer F.Cu) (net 14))
 (segment (start 129.54 73.66) (end 138.0687 82.1887) (width 0.5) (layer F.Cu) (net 14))
 (segment (start 126.972 106.5021) (end 126.972 115.19) (width 0.5) (layer F.Cu) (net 15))
 (segment (start 123.11 102.6401) (end 126.972 106.5021) (width 0.5) (layer F.Cu) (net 15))
 (segment (start 123.11 77.55) (end 123.11 102.6401) (width 0.5) (layer F.Cu) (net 15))
 (segment (start 127 73.66) (end 123.11 77.55) (width 0.5) (layer F.Cu) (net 15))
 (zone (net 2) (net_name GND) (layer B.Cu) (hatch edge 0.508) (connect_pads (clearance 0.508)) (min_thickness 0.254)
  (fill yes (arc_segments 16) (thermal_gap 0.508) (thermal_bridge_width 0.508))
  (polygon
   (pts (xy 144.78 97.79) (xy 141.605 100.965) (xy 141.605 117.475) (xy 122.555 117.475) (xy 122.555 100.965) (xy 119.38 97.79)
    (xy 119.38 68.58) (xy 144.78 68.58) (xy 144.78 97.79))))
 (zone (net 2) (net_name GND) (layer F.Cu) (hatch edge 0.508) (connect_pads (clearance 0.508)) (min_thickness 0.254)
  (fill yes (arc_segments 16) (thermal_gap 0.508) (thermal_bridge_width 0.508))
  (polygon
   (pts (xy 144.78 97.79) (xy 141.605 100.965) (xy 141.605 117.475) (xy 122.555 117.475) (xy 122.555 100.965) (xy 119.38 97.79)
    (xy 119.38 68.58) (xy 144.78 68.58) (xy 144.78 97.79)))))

